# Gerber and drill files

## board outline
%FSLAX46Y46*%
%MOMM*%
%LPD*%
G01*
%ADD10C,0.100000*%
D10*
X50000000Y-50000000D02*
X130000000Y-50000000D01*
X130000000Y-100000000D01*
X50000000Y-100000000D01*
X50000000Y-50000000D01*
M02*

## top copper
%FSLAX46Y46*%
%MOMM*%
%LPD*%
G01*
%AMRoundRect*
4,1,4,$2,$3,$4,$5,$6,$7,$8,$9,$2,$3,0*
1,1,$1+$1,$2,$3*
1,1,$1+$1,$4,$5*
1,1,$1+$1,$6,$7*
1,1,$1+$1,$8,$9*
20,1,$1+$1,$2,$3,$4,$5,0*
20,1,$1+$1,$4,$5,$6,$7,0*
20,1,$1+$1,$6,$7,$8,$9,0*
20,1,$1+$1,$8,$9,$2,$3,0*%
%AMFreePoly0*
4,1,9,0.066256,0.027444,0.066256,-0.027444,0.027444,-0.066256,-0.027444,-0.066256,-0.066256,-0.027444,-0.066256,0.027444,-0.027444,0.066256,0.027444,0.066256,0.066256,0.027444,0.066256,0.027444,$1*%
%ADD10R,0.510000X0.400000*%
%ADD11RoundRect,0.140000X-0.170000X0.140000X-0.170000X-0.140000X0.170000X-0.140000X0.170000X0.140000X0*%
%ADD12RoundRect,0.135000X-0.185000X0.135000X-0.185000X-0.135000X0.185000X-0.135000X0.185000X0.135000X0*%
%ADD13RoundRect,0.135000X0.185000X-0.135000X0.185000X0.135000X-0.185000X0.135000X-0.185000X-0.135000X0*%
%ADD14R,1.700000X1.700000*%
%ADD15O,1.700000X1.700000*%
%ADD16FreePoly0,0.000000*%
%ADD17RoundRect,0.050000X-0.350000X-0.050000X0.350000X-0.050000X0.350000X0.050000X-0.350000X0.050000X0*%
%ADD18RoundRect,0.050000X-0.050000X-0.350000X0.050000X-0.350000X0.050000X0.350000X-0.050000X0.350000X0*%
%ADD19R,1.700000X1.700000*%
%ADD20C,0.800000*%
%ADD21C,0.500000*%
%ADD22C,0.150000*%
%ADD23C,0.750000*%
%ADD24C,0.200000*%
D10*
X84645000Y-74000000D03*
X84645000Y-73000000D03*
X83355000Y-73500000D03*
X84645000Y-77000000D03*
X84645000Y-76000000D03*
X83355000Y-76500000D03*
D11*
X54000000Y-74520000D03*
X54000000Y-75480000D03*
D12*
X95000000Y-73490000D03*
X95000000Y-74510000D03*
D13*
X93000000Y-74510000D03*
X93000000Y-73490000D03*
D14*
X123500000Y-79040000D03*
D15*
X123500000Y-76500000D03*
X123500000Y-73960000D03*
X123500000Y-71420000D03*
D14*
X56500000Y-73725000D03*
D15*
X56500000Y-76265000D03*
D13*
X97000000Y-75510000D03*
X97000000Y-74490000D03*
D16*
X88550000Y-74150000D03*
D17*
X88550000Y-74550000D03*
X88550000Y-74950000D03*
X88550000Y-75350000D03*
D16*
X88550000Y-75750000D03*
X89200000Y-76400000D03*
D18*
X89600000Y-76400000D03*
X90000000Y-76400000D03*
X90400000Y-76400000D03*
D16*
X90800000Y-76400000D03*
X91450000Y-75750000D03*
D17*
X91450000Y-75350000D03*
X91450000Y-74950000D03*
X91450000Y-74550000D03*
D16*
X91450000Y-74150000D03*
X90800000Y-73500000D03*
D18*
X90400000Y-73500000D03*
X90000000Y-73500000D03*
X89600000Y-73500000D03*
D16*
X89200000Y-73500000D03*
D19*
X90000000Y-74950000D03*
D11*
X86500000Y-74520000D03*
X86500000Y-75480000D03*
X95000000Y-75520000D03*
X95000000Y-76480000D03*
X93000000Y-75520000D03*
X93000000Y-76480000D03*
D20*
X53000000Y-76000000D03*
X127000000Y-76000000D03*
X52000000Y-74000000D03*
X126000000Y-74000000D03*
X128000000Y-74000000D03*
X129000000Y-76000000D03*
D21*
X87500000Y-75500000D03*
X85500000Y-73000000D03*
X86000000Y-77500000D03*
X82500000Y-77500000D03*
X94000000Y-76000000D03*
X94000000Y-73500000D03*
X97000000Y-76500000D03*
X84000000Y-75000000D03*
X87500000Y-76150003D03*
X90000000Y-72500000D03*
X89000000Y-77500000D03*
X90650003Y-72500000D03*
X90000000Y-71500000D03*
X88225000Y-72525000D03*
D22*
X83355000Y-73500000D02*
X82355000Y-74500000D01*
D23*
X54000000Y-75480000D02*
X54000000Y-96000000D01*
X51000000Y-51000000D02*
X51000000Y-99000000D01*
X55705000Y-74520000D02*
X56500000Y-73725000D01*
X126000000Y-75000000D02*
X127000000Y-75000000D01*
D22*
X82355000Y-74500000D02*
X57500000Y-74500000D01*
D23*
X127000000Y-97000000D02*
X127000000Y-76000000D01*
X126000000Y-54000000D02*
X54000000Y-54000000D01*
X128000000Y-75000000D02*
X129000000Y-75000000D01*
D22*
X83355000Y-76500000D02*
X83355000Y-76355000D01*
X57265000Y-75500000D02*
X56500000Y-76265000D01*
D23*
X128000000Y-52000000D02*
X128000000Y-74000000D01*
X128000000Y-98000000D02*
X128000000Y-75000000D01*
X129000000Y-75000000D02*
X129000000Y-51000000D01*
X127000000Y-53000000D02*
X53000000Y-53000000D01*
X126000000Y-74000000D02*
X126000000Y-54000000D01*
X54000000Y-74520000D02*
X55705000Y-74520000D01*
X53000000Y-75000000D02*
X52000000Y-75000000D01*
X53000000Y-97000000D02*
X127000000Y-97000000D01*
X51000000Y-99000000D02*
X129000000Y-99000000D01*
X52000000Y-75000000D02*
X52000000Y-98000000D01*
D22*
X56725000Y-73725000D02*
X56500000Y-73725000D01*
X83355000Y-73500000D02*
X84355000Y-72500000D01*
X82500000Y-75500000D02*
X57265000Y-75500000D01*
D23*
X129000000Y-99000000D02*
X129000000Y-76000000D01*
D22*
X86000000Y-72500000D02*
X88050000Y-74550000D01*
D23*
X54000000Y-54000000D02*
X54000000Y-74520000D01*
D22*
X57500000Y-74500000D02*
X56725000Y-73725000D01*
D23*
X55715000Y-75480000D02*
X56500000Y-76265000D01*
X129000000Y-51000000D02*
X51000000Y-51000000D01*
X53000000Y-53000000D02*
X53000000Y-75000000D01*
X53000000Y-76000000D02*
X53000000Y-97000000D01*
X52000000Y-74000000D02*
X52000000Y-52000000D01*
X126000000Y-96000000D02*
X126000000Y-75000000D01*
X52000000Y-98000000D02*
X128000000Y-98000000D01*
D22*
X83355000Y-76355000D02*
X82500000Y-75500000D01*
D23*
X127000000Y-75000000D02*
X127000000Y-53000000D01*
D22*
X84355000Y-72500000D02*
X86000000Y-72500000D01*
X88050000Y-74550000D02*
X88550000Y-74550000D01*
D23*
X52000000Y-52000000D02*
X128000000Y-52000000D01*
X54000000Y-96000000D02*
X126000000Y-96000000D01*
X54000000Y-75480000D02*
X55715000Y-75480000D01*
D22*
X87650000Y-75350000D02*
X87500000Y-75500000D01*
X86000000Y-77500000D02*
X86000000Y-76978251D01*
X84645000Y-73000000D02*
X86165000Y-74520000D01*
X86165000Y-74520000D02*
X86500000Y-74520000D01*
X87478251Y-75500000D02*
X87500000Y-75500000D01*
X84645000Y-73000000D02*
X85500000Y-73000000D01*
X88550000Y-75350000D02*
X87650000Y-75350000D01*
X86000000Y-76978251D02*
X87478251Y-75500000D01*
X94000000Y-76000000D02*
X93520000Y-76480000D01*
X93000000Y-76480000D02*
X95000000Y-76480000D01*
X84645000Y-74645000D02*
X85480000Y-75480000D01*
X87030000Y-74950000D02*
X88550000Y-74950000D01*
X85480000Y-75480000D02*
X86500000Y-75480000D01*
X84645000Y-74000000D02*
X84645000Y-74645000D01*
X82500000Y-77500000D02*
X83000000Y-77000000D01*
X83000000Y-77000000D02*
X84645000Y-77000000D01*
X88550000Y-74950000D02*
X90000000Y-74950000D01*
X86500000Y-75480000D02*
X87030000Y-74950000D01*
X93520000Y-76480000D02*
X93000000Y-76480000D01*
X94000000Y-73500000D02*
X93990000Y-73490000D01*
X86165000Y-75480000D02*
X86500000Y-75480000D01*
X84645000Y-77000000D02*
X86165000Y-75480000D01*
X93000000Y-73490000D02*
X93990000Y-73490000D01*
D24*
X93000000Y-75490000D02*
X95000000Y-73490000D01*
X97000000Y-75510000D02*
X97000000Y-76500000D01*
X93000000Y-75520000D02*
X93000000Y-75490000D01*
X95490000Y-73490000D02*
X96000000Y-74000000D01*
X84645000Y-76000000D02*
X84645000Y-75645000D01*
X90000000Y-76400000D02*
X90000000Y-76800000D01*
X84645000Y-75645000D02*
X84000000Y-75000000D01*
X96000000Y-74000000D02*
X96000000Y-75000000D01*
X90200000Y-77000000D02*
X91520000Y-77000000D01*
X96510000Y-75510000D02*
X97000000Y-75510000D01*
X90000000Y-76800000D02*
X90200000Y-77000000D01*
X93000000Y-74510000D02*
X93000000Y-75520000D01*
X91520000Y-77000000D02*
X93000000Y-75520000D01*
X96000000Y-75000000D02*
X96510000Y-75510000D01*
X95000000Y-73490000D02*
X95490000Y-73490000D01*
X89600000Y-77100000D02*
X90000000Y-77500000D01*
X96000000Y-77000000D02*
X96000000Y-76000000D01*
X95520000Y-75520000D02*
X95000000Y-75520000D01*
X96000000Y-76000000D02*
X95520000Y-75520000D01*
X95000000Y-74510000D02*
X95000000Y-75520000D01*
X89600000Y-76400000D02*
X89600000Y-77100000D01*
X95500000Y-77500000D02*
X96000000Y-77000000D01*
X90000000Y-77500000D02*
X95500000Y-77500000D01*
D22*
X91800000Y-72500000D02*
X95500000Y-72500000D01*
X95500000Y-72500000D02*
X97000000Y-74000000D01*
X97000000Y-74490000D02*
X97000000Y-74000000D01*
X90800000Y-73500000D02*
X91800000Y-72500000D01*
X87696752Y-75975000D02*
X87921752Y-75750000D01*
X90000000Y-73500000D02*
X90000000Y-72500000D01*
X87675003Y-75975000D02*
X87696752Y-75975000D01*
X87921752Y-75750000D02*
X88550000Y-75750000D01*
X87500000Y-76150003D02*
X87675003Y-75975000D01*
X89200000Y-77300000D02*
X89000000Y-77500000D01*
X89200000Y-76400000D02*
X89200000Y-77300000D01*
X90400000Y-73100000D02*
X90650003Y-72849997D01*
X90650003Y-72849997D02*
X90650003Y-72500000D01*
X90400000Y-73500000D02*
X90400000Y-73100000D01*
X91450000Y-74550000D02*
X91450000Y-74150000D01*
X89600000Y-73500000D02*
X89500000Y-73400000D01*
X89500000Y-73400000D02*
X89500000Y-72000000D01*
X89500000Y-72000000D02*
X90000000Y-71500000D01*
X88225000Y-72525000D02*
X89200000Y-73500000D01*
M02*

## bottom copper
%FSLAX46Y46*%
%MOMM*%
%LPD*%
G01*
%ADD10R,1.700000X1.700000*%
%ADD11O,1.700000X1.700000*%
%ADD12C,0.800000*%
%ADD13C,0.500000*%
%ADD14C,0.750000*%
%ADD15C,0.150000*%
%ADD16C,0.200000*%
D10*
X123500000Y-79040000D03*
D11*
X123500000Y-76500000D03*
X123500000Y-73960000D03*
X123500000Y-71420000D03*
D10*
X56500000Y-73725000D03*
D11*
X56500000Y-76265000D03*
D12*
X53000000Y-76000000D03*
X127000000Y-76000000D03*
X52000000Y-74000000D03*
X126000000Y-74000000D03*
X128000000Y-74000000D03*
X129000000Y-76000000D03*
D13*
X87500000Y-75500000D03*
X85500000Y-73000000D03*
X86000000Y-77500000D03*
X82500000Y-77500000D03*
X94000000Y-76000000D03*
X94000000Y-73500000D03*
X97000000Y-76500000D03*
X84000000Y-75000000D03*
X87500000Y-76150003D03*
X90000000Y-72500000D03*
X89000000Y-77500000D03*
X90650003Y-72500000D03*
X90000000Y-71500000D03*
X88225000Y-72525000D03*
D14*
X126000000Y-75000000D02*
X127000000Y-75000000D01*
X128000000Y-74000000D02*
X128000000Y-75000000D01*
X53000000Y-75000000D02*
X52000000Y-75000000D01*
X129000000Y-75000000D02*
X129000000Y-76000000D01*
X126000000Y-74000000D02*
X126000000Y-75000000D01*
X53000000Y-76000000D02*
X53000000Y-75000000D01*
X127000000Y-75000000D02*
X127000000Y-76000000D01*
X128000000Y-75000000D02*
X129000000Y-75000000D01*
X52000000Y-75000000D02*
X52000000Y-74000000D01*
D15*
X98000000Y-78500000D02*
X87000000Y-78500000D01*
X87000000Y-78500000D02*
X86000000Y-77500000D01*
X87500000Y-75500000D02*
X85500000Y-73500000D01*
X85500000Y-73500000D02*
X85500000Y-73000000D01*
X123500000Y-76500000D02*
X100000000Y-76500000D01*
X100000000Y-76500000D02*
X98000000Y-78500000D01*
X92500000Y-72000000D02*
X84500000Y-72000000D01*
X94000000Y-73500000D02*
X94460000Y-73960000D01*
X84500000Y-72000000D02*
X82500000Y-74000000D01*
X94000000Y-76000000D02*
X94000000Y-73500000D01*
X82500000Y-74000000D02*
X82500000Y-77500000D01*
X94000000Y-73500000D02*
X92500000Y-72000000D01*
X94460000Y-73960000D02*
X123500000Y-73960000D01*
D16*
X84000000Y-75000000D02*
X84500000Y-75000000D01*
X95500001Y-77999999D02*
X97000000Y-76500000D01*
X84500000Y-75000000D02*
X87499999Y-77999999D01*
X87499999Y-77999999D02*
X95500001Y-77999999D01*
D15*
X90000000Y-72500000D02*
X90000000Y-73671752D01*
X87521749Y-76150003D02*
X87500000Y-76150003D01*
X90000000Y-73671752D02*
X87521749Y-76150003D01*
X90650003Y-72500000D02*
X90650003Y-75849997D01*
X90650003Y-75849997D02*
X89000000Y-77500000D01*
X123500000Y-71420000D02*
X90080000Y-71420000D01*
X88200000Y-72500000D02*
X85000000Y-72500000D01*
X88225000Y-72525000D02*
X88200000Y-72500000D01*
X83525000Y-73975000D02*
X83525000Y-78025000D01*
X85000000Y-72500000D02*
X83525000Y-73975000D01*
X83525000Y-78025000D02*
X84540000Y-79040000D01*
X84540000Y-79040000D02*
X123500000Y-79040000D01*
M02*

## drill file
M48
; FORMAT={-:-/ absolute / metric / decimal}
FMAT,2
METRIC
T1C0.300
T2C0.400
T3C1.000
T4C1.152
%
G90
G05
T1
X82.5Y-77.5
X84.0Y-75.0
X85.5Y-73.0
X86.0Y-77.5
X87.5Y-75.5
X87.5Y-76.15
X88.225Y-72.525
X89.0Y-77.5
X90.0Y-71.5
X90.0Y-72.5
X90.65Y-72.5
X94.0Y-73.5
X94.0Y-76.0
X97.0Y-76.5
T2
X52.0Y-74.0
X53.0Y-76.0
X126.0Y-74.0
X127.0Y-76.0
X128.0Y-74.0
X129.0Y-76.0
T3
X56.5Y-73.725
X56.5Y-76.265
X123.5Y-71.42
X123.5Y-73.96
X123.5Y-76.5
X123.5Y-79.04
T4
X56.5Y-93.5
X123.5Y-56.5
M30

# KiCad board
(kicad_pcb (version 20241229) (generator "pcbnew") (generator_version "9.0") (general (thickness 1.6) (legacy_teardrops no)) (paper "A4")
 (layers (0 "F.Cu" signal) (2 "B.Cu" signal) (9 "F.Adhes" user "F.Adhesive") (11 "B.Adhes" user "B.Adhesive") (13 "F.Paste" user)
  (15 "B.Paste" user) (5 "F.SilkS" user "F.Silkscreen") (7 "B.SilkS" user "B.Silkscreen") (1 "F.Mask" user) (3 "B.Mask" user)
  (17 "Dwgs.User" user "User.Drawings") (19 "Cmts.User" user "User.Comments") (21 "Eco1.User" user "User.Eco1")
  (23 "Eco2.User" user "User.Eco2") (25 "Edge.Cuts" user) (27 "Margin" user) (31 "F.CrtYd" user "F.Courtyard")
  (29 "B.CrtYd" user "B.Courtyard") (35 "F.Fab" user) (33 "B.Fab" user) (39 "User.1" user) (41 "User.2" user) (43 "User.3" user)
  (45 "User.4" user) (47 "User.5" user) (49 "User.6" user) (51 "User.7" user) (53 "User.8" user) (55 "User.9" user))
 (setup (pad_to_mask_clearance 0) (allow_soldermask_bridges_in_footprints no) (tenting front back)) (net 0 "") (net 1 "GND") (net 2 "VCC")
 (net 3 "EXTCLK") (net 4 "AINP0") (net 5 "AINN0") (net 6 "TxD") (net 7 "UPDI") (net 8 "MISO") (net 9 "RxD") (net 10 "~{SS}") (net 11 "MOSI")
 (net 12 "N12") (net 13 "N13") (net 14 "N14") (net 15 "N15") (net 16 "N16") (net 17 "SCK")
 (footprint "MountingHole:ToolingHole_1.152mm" (layer "F.Cu") (at 123.5 56.5)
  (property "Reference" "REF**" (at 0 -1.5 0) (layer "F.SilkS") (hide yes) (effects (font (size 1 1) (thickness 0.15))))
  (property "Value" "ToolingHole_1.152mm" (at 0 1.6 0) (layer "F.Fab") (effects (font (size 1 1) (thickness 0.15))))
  (pad "" np_thru_hole circle (at 0 0) (size 1.152 1.152) (drill 1.152) (layers "*.Cu" "*.Mask") (solder_mask_margin 0.074))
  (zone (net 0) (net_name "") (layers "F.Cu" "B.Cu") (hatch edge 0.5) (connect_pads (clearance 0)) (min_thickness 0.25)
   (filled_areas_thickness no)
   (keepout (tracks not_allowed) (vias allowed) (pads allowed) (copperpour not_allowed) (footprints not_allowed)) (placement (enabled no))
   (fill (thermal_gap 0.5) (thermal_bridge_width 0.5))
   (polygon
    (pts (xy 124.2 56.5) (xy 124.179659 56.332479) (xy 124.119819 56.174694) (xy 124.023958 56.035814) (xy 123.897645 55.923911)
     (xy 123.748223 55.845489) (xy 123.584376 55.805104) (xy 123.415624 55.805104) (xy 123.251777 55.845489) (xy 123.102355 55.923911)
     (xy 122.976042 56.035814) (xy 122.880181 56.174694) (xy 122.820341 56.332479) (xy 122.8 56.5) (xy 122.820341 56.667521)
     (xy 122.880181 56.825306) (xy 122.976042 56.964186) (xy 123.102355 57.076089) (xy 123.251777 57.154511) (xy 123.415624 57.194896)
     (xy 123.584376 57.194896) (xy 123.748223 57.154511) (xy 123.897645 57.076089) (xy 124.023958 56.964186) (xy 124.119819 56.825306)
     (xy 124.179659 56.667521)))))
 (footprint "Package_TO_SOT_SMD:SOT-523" (layer "F.Cu") (at 84 73.5 180)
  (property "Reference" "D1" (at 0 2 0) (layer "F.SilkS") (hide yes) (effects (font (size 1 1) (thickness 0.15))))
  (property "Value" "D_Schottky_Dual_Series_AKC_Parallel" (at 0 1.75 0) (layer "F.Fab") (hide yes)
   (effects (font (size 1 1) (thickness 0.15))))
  (pad "1" smd rect (at -0.645 -0.5) (size 0.51 0.4) (layers "F.Cu" "F.Mask" "F.Paste") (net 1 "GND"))
  (pad "2" smd rect (at -0.645 0.5) (size 0.51 0.4) (layers "F.Cu" "F.Mask" "F.Paste") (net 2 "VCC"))
  (pad "3" smd rect (at 0.645 0) (size 0.51 0.4) (layers "F.Cu" "F.Mask" "F.Paste") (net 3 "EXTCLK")))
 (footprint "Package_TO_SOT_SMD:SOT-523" (layer "F.Cu") (at 84 76.5 180)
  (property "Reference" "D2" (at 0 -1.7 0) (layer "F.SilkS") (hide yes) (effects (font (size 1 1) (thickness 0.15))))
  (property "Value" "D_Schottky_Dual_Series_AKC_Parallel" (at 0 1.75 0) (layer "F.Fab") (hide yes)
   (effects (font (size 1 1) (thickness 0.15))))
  (pad "1" smd rect (at -0.645 -0.5) (size 0.51 0.4) (layers "F.Cu" "F.Mask" "F.Paste") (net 1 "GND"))
  (pad "2" smd rect (at -0.645 0.5) (size 0.51 0.4) (layers "F.Cu" "F.Mask" "F.Paste") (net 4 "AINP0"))
  (pad "3" smd rect (at 0.645 0) (size 0.51 0.4) (layers "F.Cu" "F.Mask" "F.Paste") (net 3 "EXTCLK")))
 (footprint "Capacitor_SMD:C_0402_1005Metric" (layer "F.Cu") (at 54 75 -90)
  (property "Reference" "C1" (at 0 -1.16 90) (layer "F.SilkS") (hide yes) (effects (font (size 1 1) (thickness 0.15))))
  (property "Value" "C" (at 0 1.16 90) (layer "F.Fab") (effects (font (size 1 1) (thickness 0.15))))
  (pad "1" smd roundrect (at -0.48 0 270) (size 0.56 0.62) (layers "F.Cu" "F.Mask" "F.Paste") (roundrect_rratio 0.25) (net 3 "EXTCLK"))
  (pad "2" smd roundrect (at 0.48 0 270) (size 0.56 0.62) (layers "F.Cu" "F.Mask" "F.Paste") (roundrect_rratio 0.25) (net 3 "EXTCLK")))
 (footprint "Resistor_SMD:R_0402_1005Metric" (layer "F.Cu") (at 95 74 -90)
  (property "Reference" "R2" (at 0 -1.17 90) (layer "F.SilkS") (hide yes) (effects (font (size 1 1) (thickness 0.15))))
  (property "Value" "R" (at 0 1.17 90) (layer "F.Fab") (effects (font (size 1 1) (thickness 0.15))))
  (pad "1" smd roundrect (at -0.51 0 270) (size 0.54 0.64) (layers "F.Cu" "F.Mask" "F.Paste") (roundrect_rratio 0.25) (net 4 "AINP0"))
  (pad "2" smd roundrect (at 0.51 0 270) (size 0.54 0.64) (layers "F.Cu" "F.Mask" "F.Paste") (roundrect_rratio 0.25) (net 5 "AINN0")))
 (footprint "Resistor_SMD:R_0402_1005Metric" (layer "F.Cu") (at 93 74 90)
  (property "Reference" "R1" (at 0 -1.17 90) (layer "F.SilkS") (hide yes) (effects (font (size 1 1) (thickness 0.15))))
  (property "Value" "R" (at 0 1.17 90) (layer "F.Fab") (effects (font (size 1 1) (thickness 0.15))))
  (pad "1" smd roundrect (at -0.51 0 90) (size 0.54 0.64) (layers "F.Cu" "F.Mask" "F.Paste") (roundrect_rratio 0.25) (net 4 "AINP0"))
  (pad "2" smd roundrect (at 0.51 0 90) (size 0.54 0.64) (layers "F.Cu" "F.Mask" "F.Paste") (roundrect_rratio 0.25) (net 1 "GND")))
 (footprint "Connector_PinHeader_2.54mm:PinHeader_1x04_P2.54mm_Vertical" (layer "F.Cu") (at 123.5 79.04 180)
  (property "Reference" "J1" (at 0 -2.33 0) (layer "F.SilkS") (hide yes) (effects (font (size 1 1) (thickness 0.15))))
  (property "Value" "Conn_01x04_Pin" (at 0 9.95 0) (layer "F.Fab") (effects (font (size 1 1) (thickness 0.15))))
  (pad "1" thru_hole rect (at 0 0 180) (size 1.7 1.7) (drill 1) (layers "*.Cu" "*.Mask") (remove_unused_layers no) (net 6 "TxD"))
  (pad "2" thru_hole oval (at 0 2.54 180) (size 1.7 1.7) (drill 1) (layers "*.Cu" "*.Mask") (remove_unused_layers no) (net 2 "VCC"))
  (pad "3" thru_hole oval (at 0 5.08 180) (size 1.7 1.7) (drill 1) (layers "*.Cu" "*.Mask") (remove_unused_layers no) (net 1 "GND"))
  (pad "4" thru_hole oval (at 0 7.62 180) (size 1.7 1.7) (drill 1) (layers "*.Cu" "*.Mask") (remove_unused_layers no) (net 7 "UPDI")))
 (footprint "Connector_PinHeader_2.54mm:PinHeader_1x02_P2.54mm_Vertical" (layer "F.Cu") (at 56.5 73.725)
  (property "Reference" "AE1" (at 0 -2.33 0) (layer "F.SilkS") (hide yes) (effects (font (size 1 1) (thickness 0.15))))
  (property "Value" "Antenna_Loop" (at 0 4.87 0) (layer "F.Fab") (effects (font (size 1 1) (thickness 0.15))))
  (pad "1" thru_hole rect (at 0 0) (size 1.7 1.7) (drill 1) (layers "*.Cu" "*.Mask") (remove_unused_layers no) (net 3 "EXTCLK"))
  (pad "2" thru_hole oval (at 0 2.54) (size 1.7 1.7) (drill 1) (layers "*.Cu" "*.Mask") (remove_unused_layers no) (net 3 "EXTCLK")))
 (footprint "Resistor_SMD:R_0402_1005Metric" (layer "F.Cu") (at 97 75 90)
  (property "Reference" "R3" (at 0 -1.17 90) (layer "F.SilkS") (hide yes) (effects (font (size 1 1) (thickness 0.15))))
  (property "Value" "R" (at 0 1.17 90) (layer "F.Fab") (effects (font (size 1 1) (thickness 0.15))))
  (pad "1" smd roundrect (at -0.51 0 90) (size 0.54 0.64) (layers "F.Cu" "F.Mask" "F.Paste") (roundrect_rratio 0.25) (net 4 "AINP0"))
  (pad "2" smd roundrect (at 0.51 0 90) (size 0.54 0.64) (layers "F.Cu" "F.Mask" "F.Paste") (roundrect_rratio 0.25) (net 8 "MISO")))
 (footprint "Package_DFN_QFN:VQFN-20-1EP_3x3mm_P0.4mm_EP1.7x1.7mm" (layer "F.Cu") (at 90 74.95)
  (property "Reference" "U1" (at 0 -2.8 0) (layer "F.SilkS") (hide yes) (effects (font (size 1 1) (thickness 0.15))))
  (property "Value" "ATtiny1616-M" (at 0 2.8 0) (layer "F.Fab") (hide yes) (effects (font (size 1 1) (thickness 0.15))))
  (pad "" smd roundrect (at -0.425 -0.425) (size 0.69 0.69) (layers "F.Paste") (roundrect_rratio 0.25))
  (pad "" smd roundrect (at -0.425 0.425) (size 0.69 0.69) (layers "F.Paste") (roundrect_rratio 0.25))
  (pad "" smd roundrect (at 0.425 -0.425) (size 0.69 0.69) (layers "F.Paste") (roundrect_rratio 0.25))
  (pad "" smd roundrect (at 0.425 0.425) (size 0.69 0.69) (layers "F.Paste") (roundrect_rratio 0.25))
  (pad "1" smd custom (at -1.45 -0.8) (size 0.143431 0.143431) (layers "F.Cu" "F.Mask" "F.Paste") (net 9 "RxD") (thermal_bridge_angle 90)
   (options (clearance outline) (anchor circle)) (primitives))
  (pad "2" smd roundrect (at -1.45 -0.4) (size 0.8 0.2) (layers "F.Cu" "F.Mask" "F.Paste") (roundrect_rratio 0.25) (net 3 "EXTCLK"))
  (pad "3" smd roundrect (at -1.45 0) (size 0.8 0.2) (layers "F.Cu" "F.Mask" "F.Paste") (roundrect_rratio 0.25) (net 1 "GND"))
  (pad "4" smd roundrect (at -1.45 0.4) (size 0.8 0.2) (layers "F.Cu" "F.Mask" "F.Paste") (roundrect_rratio 0.25) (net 2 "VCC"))
  (pad "5" smd custom (at -1.45 0.8) (size 0.143431 0.143431) (layers "F.Cu" "F.Mask" "F.Paste") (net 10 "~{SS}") (thermal_bridge_angle 90)
   (options (clearance outline) (anchor circle)) (primitives))
  (pad "6" smd custom (at -0.8 1.45) (size 0.143431 0.143431) (layers "F.Cu" "F.Mask" "F.Paste") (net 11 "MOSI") (thermal_bridge_angle 90)
   (options (clearance outline) (anchor circle)) (primitives))
  (pad "7" smd roundrect (at -0.4 1.45) (size 0.2 0.8) (layers "F.Cu" "F.Mask" "F.Paste") (roundrect_rratio 0.25) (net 5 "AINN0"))
  (pad "8" smd roundrect (at 0 1.45) (size 0.2 0.8) (layers "F.Cu" "F.Mask" "F.Paste") (roundrect_rratio 0.25) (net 4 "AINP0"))
  (pad "9" smd roundrect (at 0.4 1.45) (size 0.2 0.8) (layers "F.Cu" "F.Mask" "F.Paste") (roundrect_rratio 0.25) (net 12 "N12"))
  (pad "10" smd custom (at 0.8 1.45) (size 0.143431 0.143431) (layers "F.Cu" "F.Mask" "F.Paste") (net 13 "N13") (thermal_bridge_angle 90)
   (options (clearance outline) (anchor circle)) (primitives))
  (pad "11" smd custom (at 1.45 0.8) (size 0.143431 0.143431) (layers "F.Cu" "F.Mask" "F.Paste") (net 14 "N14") (thermal_bridge_angle 90)
   (options (clearance outline) (anchor circle)) (primitives))
  (pad "12" smd roundrect (at 1.45 0.4) (size 0.8 0.2) (layers "F.Cu" "F.Mask" "F.Paste") (roundrect_rratio 0.25) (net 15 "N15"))
  (pad "13" smd roundrect (at 1.45 0) (size 0.8 0.2) (layers "F.Cu" "F.Mask" "F.Paste") (roundrect_rratio 0.25) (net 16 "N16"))
  (pad "14" smd roundrect (at 1.45 -0.4) (size 0.8 0.2) (layers "F.Cu" "F.Mask" "F.Paste") (roundrect_rratio 0.25) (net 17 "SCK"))
  (pad "15" smd custom (at 1.45 -0.8) (size 0.143431 0.143431) (layers "F.Cu" "F.Mask" "F.Paste") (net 17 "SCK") (thermal_bridge_angle 90)
   (options (clearance outline) (anchor circle)) (primitives))
  (pad "16" smd custom (at 0.8 -1.45) (size 0.143431 0.143431) (layers "F.Cu" "F.Mask" "F.Paste") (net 8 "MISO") (thermal_bridge_angle 90)
   (options (clearance outline) (anchor circle)) (primitives))
  (pad "17" smd roundrect (at 0.4 -1.45) (size 0.2 0.8) (layers "F.Cu" "F.Mask" "F.Paste") (roundrect_rratio 0.25) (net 11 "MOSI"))
  (pad "18" smd roundrect (at 0 -1.45) (size 0.2 0.8) (layers "F.Cu" "F.Mask" "F.Paste") (roundrect_rratio 0.25) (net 10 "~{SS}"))
  (pad "19" smd roundrect (at -0.4 -1.45) (size 0.2 0.8) (layers "F.Cu" "F.Mask" "F.Paste") (roundrect_rratio 0.25) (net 7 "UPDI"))
  (pad "20" smd custom (at -0.8 -1.45) (size 0.143431 0.143431) (layers "F.Cu" "F.Mask" "F.Paste") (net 6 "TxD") (thermal_bridge_angle 90)
   (options (clearance outline) (anchor circle)) (primitives))
  (pad "21" smd rect (at 0 0) (size 1.7 1.7) (layers "F.Cu" "F.Mask") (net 1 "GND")))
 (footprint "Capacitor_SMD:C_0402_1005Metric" (layer "F.Cu") (at 86.5 75 -90)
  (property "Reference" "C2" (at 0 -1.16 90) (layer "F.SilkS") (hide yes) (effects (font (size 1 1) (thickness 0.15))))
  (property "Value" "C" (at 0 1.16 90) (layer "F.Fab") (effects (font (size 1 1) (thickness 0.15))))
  (pad "1" smd roundrect (at -0.48 0 270) (size 0.56 0.62) (layers "F.Cu" "F.Mask" "F.Paste") (roundrect_rratio 0.25) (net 2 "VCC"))
  (pad "2" smd roundrect (at 0.48 0 270) (size 0.56 0.62) (layers "F.Cu" "F.Mask" "F.Paste") (roundrect_rratio 0.25) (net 1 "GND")))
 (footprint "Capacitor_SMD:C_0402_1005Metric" (layer "F.Cu") (at 95 76 -90)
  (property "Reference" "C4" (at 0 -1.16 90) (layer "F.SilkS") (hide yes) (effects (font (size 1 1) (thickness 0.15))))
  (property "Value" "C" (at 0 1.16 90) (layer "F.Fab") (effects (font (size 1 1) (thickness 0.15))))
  (pad "1" smd roundrect (at -0.48 0 270) (size 0.56 0.62) (layers "F.Cu" "F.Mask" "F.Paste") (roundrect_rratio 0.25) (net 5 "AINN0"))
  (pad "2" smd roundrect (at 0.48 0 270) (size 0.56 0.62) (layers "F.Cu" "F.Mask" "F.Paste") (roundrect_rratio 0.25) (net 1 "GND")))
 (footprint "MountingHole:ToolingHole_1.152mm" (layer "F.Cu") (at 56.5 93.5)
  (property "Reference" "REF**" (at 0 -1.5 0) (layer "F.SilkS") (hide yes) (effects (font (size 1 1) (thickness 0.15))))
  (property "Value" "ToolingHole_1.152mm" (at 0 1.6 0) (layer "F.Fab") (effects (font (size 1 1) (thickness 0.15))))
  (pad "" np_thru_hole circle (at 0 0) (size 1.152 1.152) (drill 1.152) (layers "*.Cu" "*.Mask") (solder_mask_margin 0.074))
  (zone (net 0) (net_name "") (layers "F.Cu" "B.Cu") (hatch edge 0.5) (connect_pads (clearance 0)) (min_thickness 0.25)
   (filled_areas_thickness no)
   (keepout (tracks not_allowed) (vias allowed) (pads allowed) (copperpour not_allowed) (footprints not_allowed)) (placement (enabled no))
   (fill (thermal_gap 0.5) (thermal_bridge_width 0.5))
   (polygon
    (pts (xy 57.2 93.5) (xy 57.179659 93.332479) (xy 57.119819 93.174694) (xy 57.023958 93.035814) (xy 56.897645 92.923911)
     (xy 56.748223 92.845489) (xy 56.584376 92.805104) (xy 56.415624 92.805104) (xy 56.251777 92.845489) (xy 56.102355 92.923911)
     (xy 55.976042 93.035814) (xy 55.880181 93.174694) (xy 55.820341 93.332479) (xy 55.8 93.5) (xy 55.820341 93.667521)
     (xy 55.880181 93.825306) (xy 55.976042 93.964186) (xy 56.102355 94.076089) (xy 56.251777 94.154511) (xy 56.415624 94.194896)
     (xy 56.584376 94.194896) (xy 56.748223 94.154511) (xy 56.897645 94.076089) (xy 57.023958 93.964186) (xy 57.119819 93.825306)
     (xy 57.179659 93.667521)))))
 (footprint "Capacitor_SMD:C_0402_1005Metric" (layer "F.Cu") (at 93 76 -90)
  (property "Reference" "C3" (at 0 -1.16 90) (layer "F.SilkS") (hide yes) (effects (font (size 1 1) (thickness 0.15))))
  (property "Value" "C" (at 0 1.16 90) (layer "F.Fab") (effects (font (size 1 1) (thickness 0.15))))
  (pad "1" smd roundrect (at -0.48 0 270) (size 0.56 0.62) (layers "F.Cu" "F.Mask" "F.Paste") (roundrect_rratio 0.25) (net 4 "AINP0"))
  (pad "2" smd roundrect (at 0.48 0 270) (size 0.56 0.62) (layers "F.Cu" "F.Mask" "F.Paste") (roundrect_rratio 0.25) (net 1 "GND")))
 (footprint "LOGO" (layer "B.Cu") (at 90 75 180)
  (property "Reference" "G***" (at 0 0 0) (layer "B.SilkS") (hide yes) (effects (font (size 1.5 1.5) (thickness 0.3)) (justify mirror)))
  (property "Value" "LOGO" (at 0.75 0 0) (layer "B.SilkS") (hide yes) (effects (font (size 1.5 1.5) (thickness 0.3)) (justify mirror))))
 (gr_rect (start 50 50) (end 130 100) (stroke (width 0.1) (type default)) (fill no) (locked yes) (layer "Edge.Cuts"))
 (segment (start 83.355 73.5) (end 82.355 74.5) (width 0.15) (layer "F.Cu") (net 3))
 (segment (start 54 75.48) (end 54 96) (width 0.75) (layer "F.Cu") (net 3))
 (segment (start 51 51) (end 51 99) (width 0.75) (layer "F.Cu") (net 3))
 (segment (start 55.705 74.52) (end 56.5 73.725) (width 0.75) (layer "F.Cu") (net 3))
 (segment (start 126 75) (end 127 75) (width 0.75) (layer "F.Cu") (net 3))
 (segment (start 82.355 74.5) (end 57.5 74.5) (width 0.15) (layer "F.Cu") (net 3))
 (segment (start 127 97) (end 127 76) (width 0.75) (layer "F.Cu") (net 3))
 (segment (start 126 54) (end 54 54) (width 0.75) (layer "F.Cu") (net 3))
 (segment (start 128 75) (end 129 75) (width 0.75) (layer "F.Cu") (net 3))
 (segment (start 83.355 76.5) (end 83.355 76.355) (width 0.15) (layer "F.Cu") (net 3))
 (segment (start 57.265 75.5) (end 56.5 76.265) (width 0.15) (layer "F.Cu") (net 3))
 (segment (start 128 52) (end 128 74) (width 0.75) (layer "F.Cu") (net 3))
 (segment (start 128 98) (end 128 75) (width 0.75) (layer "F.Cu") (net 3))
 (segment (start 129 75) (end 129 51) (width 0.75) (layer "F.Cu") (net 3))
 (segment (start 127 53) (end 53 53) (width 0.75) (layer "F.Cu") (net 3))
 (segment (start 126 74) (end 126 54) (width 0.75) (layer "F.Cu") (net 3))
 (segment (start 54 74.52) (end 55.705 74.52) (width 0.75) (layer "F.Cu") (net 3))
 (segment (start 53 75) (end 52 75) (width 0.75) (layer "F.Cu") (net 3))
 (segment (start 53 97) (end 127 97) (width 0.75) (layer "F.Cu") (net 3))
 (segment (start 51 99) (end 129 99) (width 0.75) (layer "F.Cu") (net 3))
 (segment (start 52 75) (end 52 98) (width 0.75) (layer "F.Cu") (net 3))
 (segment (start 56.725 73.725) (end 56.5 73.725) (width 0.15) (layer "F.Cu") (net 3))
 (segment (start 83.355 73.5) (end 84.355 72.5) (width 0.15) (layer "F.Cu") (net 3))
 (segment (start 82.5 75.5) (end 57.265 75.5) (width 0.15) (layer "F.Cu") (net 3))
 (segment (start 129 99) (end 129 76) (width 0.75) (layer "F.Cu") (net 3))
 (segment (start 86 72.5) (end 88.05 74.55) (width 0.15) (layer "F.Cu") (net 3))
 (segment (start 54 54) (end 54 74.52) (width 0.75) (layer "F.Cu") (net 3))
 (segment (start 57.5 74.5) (end 56.725 73.725) (width 0.15) (layer "F.Cu") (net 3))
 (segment (start 55.715 75.48) (end 56.5 76.265) (width 0.75) (layer "F.Cu") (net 3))
 (segment (start 129 51) (end 51 51) (width 0.75) (layer "F.Cu") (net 3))
 (segment (start 53 53) (end 53 75) (width 0.75) (layer "F.Cu") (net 3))
 (segment (start 53 76) (end 53 97) (width 0.75) (layer "F.Cu") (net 3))
 (segment (start 52 74) (end 52 52) (width 0.75) (layer "F.Cu") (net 3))
 (segment (start 126 96) (end 126 75) (width 0.75) (layer "F.Cu") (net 3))
 (segment (start 52 98) (end 128 98) (width 0.75) (layer "F.Cu") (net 3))
 (segment (start 83.355 76.355) (end 82.5 75.5) (width 0.15) (layer "F.Cu") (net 3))
 (segment (start 127 75) (end 127 53) (width 0.75) (layer "F.Cu") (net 3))
 (segment (start 84.355 72.5) (end 86 72.5) (width 0.15) (layer "F.Cu") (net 3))
 (segment (start 88.05 74.55) (end 88.55 74.55) (width 0.15) (layer "F.Cu") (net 3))
 (segment (start 52 52) (end 128 52) (width 0.75) (layer "F.Cu") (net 3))
 (segment (start 54 96) (end 126 96) (width 0.75) (layer "F.Cu") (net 3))
 (segment (start 54 75.48) (end 55.715 75.48) (width 0.75) (layer "F.Cu") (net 3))
 (via (at 53 76) (size 0.8) (drill 0.4) (layers "F.Cu" "B.Cu") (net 3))
 (via (at 127 76) (size 0.8) (drill 0.4) (layers "F.Cu" "B.Cu") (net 3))
 (via (at 52 74) (size 0.8) (drill 0.4) (layers "F.Cu" "B.Cu") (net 3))
 (via (at 126 74) (size 0.8) (drill 0.4) (layers "F.Cu" "B.Cu") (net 3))
 (via (at 128 74) (size 0.8) (drill 0.4) (layers "F.Cu" "B.Cu") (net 3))
 (via (at 129 76) (size 0.8) (drill 0.4) (layers "F.Cu" "B.Cu") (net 3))
 (segment (start 126 75) (end 127 75) (width 0.75) (layer "B.Cu") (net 3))
 (segment (start 128 74) (end 128 75) (width 0.75) (layer "B.Cu") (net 3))
 (segment (start 53 75) (end 52 75) (width 0.75) (layer "B.Cu") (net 3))
 (segment (start 129 75) (end 129 76) (width 0.75) (layer "B.Cu") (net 3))
 (segment (start 126 74) (end 126 75) (width 0.75) (layer "B.Cu") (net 3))
 (segment (start 53 76) (end 53 75) (width 0.75) (layer "B.Cu") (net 3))
 (segment (start 127 75) (end 127 76) (width 0.75) (layer "B.Cu") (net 3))
 (segment (start 128 75) (end 129 75) (width 0.75) (layer "B.Cu") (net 3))
 (segment (start 52 75) (end 52 74) (width 0.75) (layer "B.Cu") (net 3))
 (segment (start 87.65 75.35) (end 87.5 75.5) (width 0.15) (layer "F.Cu") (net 2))
 (segment (start 86 77.5) (end 86 76.978251) (width 0.15) (layer "F.Cu") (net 2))
 (segment (start 84.645 73) (end 86.165 74.52) (width 0.15) (layer "F.Cu") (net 2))
 (segment (start 86.165 74.52) (end 86.5 74.52) (width 0.15) (layer "F.Cu") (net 2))
 (segment (start 87.478251 75.5) (end 87.5 75.5) (width 0.15) (layer "F.Cu") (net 2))
 (segment (start 84.645 73) (end 85.5 73) (width 0.15) (layer "F.Cu") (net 2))
 (segment (start 88.55 75.35) (end 87.65 75.35) (width 0.15) (layer "F.Cu") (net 2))
 (segment (start 86 76.978251) (end 87.478251 75.5) (width 0.15) (layer "F.Cu") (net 2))
 (via (at 87.5 75.5) (size 0.5) (drill 0.3) (layers "F.Cu" "B.Cu") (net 2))
 (via (at 85.5 73) (size 0.5) (drill 0.3) (layers "F.Cu" "B.Cu") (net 2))
 (via (at 86 77.5) (size 0.5) (drill 0.3) (layers "F.Cu" "B.Cu") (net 2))
 (segment (start 98 78.5) (end 87 78.5) (width 0.15) (layer "B.Cu") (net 2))
 (segment (start 87 78.5) (end 86 77.5) (width 0.15) (layer "B.Cu") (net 2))
 (segment (start 87.5 75.5) (end 85.5 73.5) (width 0.15) (layer "B.Cu") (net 2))
 (segment (start 85.5 73.5) (end 85.5 73) (width 0.15) (layer "B.Cu") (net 2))
 (segment (start 123.5 76.5) (end 100 76.5) (width 0.15) (layer "B.Cu") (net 2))
 (segment (start 100 76.5) (end 98 78.5) (width 0.15) (layer "B.Cu") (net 2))
 (segment (start 94 76) (end 93.52 76.48) (width 0.15) (layer "F.Cu") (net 1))
 (segment (start 93 76.48) (end 95 76.48) (width 0.15) (layer "F.Cu") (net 1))
 (segment (start 84.645 74.645) (end 85.48 75.48) (width 0.15) (layer "F.Cu") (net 1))
 (segment (start 87.03 74.95) (end 88.55 74.95) (width 0.15) (layer "F.Cu") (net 1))
 (segment (start 85.48 75.48) (end 86.5 75.48) (width 0.15) (layer "F.Cu") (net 1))
 (segment (start 84.645 74) (end 84.645 74.645) (width 0.15) (layer "F.Cu") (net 1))
 (segment (start 82.5 77.5) (end 83 77) (width 0.15) (layer "F.Cu") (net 1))
 (segment (start 83 77) (end 84.645 77) (width 0.15) (layer "F.Cu") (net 1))
 (segment (start 88.55 74.95) (end 90 74.95) (width 0.15) (layer "F.Cu") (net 1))
 (segment (start 86.5 75.48) (end 87.03 74.95) (width 0.15) (layer "F.Cu") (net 1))
 (segment (start 93.52 76.48) (end 93 76.48) (width 0.15) (layer "F.Cu") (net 1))
 (segment (start 94 73.5) (end 93.99 73.49) (width 0.15) (layer "F.Cu") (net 1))
 (segment (start 86.165 75.48) (end 86.5 75.48) (width 0.15) (layer "F.Cu") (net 1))
 (segment (start 84.645 77) (end 86.165 75.48) (width 0.15) (layer "F.Cu") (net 1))
 (segment (start 93 73.49) (end 93.99 73.49) (width 0.15) (layer "F.Cu") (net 1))
 (via (at 82.5 77.5) (size 0.5) (drill 0.3) (layers "F.Cu" "B.Cu") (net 1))
 (via (at 94 76) (size 0.5) (drill 0.3) (layers "F.Cu" "B.Cu") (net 1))
 (via (at 94 73.5) (size 0.5) (drill 0.3) (layers "F.Cu" "B.Cu") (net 1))
 (segment (start 92.5 72) (end 84.5 72) (width 0.15) (layer "B.Cu") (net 1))
 (segment (start 94 73.5) (end 94.46 73.96) (width 0.15) (layer "B.Cu") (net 1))
 (segment (start 84.5 72) (end 82.5 74) (width 0.15) (layer "B.Cu") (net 1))
 (segment (start 94 76) (end 94 73.5) (width 0.15) (layer "B.Cu") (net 1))
 (segment (start 82.5 74) (end 82.5 77.5) (width 0.15) (layer "B.Cu") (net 1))
 (segment (start 94 73.5) (end 92.5 72) (width 0.15) (layer "B.Cu") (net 1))
 (segment (start 94.46 73.96) (end 123.5 73.96) (width 0.15) (layer "B.Cu") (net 1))
 (segment (start 93 75.49) (end 95 73.49) (width 0.2) (layer "F.Cu") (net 4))
 (segment (start 97 75.51) (end 97 76.5) (width 0.2) (layer "F.Cu") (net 4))
 (segment (start 93 75.52) (end 93 75.49) (width 0.2) (layer "F.Cu") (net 4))
 (segment (start 95.49 73.49) (end 96 74) (width 0.2) (layer "F.Cu") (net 4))
 (segment (start 84.645 76) (end 84.645 75.645) (width 0.2) (layer "F.Cu") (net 4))
 (segment (start 90 76.4) (end 90 76.8) (width 0.2) (layer "F.Cu") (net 4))
 (segment (start 84.645 75.645) (end 84 75) (width 0.2) (layer "F.Cu") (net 4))
 (segment (start 96 74) (end 96 75) (width 0.2) (layer "F.Cu") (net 4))
 (segment (start 90.2 77) (end 91.52 77) (width 0.2) (layer "F.Cu") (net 4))
 (segment (start 96.51 75.51) (end 97 75.51) (width 0.2) (layer "F.Cu") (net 4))
 (segment (start 90 76.8) (end 90.2 77) (width 0.2) (layer "F.Cu") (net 4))
 (segment (start 93 74.51) (end 93 75.52) (width 0.2) (layer "F.Cu") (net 4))
 (segment (start 91.52 77) (end 93 75.52) (width 0.2) (layer "F.Cu") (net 4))
 (segment (start 96 75) (end 96.51 75.51) (width 0.2) (layer "F.Cu") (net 4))
 (segment (start 95 73.49) (end 95.49 73.49) (width 0.2) (layer "F.Cu") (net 4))
 (via (at 97 76.5) (size 0.5) (drill 0.3) (layers "F.Cu" "B.Cu") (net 4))
 (via (at 84 75) (size 0.5) (drill 0.3) (layers "F.Cu" "B.Cu") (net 4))
 (segment (start 84 75) (end 84.5 75) (width 0.2) (layer "B.Cu") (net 4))
 (segment (start 95.500001 77.999999) (end 97 76.5) (width 0.2) (layer "B.Cu") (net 4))
 (segment (start 84.5 75) (end 87.499999 77.999999) (width 0.2) (layer "B.Cu") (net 4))
 (segment (start 87.499999 77.999999) (end 95.500001 77.999999) (width 0.2) (layer "B.Cu") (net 4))
 (segment (start 89.6 77.1) (end 90 77.5) (width 0.2) (layer "F.Cu") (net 5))
 (segment (start 96 77) (end 96 76) (width 0.2) (layer "F.Cu") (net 5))
 (segment (start 95.52 75.52) (end 95 75.52) (width 0.2) (layer "F.Cu") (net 5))
 (segment (start 96 76) (end 95.52 75.52) (width 0.2) (layer "F.Cu") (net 5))
 (segment (start 95 74.51) (end 95 75.52) (width 0.2) (layer "F.Cu") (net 5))
 (segment (start 89.6 76.4) (end 89.6 77.1) (width 0.2) (layer "F.Cu") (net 5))
 (segment (start 95.5 77.5) (end 96 77) (width 0.2) (layer "F.Cu") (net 5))
 (segment (start 90 77.5) (end 95.5 77.5) (width 0.2) (layer "F.Cu") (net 5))
 (segment (start 91.8 72.5) (end 95.5 72.5) (width 0.15) (layer "F.Cu") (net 8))
 (segment (start 95.5 72.5) (end 97 74) (width 0.15) (layer "F.Cu") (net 8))
 (segment (start 97 74.49) (end 97 74) (width 0.15) (layer "F.Cu") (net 8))
 (segment (start 90.8 73.5) (end 91.8 72.5) (width 0.15) (layer "F.Cu") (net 8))
 (segment (start 87.696752 75.975) (end 87.921752 75.75) (width 0.15) (layer "F.Cu") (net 10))
 (segment (start 90 73.5) (end 90 72.5) (width 0.15) (layer "F.Cu") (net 10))
 (segment (start 87.675003 75.975) (end 87.696752 75.975) (width 0.15) (layer "F.Cu") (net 10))
 (segment (start 87.921752 75.75) (end 88.55 75.75) (width 0.15) (layer "F.Cu") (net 10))
 (segment (start 87.5 76.150003) (end 87.675003 75.975) (width 0.15) (layer "F.Cu") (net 10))
 (via (at 87.5 76.150003) (size 0.5) (drill 0.3) (layers "F.Cu" "B.Cu") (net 10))
 (via (at 90 72.5) (size 0.5) (drill 0.3) (layers "F.Cu" "B.Cu") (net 10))
 (segment (start 90 72.5) (end 90 73.671752) (width 0.15) (layer "B.Cu") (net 10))
 (segment (start 87.521749 76.150003) (end 87.5 76.150003) (width 0.15) (layer "B.Cu") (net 10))
 (segment (start 90 73.671752) (end 87.521749 76.150003) (width 0.15) (layer "B.Cu") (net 10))
 (segment (start 89.2 77.3) (end 89 77.5) (width 0.15) (layer "F.Cu") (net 11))
 (segment (start 89.2 76.4) (end 89.2 77.3) (width 0.15) (layer "F.Cu") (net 11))
 (segment (start 90.4 73.1) (end 90.650003 72.849997) (width 0.15) (layer "F.Cu") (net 11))
 (segment (start 90.650003 72.849997) (end 90.650003 72.5) (width 0.15) (layer "F.Cu") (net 11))
 (segment (start 90.4 73.5) (end 90.4 73.1) (width 0.15) (layer "F.Cu") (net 11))
 (via (at 89 77.5) (size 0.5) (drill 0.3) (layers "F.Cu" "B.Cu") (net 11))
 (via (at 90.650003 72.5) (size 0.5) (drill 0.3) (layers "F.Cu" "B.Cu") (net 11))
 (segment (start 90.650003 72.5) (end 90.650003 75.849997) (width 0.15) (layer "B.Cu") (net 11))
 (segment (start 90.650003 75.849997) (end 89 77.5) (width 0.15) (layer "B.Cu") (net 11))
 (segment (start 91.45 74.55) (end 91.45 74.15) (width 0.15) (layer "F.Cu") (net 17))
 (segment (start 89.6 73.5) (end 89.5 73.4) (width 0.15) (layer "F.Cu") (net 7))
 (segment (start 89.5 73.4) (end 89.5 72) (width 0.15) (layer "F.Cu") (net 7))
 (segment (start 89.5 72) (end 90 71.5) (width 0.15) (layer "F.Cu") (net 7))
 (via (at 90 71.5) (size 0.5) (drill 0.3) (layers "F.Cu" "B.Cu") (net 7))
 (segment (start 123.5 71.42) (end 90.08 71.42) (width 0.15) (layer "B.Cu") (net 7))
 (segment (start 88.225 72.525) (end 89.2 73.5) (width 0.15) (layer "F.Cu") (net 6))
 (via (at 88.225 72.525) (size 0.5) (drill 0.3) (layers "F.Cu" "B.Cu") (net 6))
 (segment (start 88.2 72.5) (end 85 72.5) (width 0.15) (layer "B.Cu") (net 6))
 (segment (start 88.225 72.525) (end 88.2 72.5) (width 0.15) (layer "B.Cu") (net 6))
 (segment (start 83.525 73.975) (end 83.525 78.025) (width 0.15) (layer "B.Cu") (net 6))
 (segment (start 85 72.5) (end 83.525 73.975) (width 0.15) (layer "B.Cu") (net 6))
 (segment (start 83.525 78.025) (end 84.54 79.04) (width 0.15) (layer "B.Cu") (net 6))
 (segment (start 84.54 79.04) (end 123.5 79.04) (width 0.15) (layer "B.Cu") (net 6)))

